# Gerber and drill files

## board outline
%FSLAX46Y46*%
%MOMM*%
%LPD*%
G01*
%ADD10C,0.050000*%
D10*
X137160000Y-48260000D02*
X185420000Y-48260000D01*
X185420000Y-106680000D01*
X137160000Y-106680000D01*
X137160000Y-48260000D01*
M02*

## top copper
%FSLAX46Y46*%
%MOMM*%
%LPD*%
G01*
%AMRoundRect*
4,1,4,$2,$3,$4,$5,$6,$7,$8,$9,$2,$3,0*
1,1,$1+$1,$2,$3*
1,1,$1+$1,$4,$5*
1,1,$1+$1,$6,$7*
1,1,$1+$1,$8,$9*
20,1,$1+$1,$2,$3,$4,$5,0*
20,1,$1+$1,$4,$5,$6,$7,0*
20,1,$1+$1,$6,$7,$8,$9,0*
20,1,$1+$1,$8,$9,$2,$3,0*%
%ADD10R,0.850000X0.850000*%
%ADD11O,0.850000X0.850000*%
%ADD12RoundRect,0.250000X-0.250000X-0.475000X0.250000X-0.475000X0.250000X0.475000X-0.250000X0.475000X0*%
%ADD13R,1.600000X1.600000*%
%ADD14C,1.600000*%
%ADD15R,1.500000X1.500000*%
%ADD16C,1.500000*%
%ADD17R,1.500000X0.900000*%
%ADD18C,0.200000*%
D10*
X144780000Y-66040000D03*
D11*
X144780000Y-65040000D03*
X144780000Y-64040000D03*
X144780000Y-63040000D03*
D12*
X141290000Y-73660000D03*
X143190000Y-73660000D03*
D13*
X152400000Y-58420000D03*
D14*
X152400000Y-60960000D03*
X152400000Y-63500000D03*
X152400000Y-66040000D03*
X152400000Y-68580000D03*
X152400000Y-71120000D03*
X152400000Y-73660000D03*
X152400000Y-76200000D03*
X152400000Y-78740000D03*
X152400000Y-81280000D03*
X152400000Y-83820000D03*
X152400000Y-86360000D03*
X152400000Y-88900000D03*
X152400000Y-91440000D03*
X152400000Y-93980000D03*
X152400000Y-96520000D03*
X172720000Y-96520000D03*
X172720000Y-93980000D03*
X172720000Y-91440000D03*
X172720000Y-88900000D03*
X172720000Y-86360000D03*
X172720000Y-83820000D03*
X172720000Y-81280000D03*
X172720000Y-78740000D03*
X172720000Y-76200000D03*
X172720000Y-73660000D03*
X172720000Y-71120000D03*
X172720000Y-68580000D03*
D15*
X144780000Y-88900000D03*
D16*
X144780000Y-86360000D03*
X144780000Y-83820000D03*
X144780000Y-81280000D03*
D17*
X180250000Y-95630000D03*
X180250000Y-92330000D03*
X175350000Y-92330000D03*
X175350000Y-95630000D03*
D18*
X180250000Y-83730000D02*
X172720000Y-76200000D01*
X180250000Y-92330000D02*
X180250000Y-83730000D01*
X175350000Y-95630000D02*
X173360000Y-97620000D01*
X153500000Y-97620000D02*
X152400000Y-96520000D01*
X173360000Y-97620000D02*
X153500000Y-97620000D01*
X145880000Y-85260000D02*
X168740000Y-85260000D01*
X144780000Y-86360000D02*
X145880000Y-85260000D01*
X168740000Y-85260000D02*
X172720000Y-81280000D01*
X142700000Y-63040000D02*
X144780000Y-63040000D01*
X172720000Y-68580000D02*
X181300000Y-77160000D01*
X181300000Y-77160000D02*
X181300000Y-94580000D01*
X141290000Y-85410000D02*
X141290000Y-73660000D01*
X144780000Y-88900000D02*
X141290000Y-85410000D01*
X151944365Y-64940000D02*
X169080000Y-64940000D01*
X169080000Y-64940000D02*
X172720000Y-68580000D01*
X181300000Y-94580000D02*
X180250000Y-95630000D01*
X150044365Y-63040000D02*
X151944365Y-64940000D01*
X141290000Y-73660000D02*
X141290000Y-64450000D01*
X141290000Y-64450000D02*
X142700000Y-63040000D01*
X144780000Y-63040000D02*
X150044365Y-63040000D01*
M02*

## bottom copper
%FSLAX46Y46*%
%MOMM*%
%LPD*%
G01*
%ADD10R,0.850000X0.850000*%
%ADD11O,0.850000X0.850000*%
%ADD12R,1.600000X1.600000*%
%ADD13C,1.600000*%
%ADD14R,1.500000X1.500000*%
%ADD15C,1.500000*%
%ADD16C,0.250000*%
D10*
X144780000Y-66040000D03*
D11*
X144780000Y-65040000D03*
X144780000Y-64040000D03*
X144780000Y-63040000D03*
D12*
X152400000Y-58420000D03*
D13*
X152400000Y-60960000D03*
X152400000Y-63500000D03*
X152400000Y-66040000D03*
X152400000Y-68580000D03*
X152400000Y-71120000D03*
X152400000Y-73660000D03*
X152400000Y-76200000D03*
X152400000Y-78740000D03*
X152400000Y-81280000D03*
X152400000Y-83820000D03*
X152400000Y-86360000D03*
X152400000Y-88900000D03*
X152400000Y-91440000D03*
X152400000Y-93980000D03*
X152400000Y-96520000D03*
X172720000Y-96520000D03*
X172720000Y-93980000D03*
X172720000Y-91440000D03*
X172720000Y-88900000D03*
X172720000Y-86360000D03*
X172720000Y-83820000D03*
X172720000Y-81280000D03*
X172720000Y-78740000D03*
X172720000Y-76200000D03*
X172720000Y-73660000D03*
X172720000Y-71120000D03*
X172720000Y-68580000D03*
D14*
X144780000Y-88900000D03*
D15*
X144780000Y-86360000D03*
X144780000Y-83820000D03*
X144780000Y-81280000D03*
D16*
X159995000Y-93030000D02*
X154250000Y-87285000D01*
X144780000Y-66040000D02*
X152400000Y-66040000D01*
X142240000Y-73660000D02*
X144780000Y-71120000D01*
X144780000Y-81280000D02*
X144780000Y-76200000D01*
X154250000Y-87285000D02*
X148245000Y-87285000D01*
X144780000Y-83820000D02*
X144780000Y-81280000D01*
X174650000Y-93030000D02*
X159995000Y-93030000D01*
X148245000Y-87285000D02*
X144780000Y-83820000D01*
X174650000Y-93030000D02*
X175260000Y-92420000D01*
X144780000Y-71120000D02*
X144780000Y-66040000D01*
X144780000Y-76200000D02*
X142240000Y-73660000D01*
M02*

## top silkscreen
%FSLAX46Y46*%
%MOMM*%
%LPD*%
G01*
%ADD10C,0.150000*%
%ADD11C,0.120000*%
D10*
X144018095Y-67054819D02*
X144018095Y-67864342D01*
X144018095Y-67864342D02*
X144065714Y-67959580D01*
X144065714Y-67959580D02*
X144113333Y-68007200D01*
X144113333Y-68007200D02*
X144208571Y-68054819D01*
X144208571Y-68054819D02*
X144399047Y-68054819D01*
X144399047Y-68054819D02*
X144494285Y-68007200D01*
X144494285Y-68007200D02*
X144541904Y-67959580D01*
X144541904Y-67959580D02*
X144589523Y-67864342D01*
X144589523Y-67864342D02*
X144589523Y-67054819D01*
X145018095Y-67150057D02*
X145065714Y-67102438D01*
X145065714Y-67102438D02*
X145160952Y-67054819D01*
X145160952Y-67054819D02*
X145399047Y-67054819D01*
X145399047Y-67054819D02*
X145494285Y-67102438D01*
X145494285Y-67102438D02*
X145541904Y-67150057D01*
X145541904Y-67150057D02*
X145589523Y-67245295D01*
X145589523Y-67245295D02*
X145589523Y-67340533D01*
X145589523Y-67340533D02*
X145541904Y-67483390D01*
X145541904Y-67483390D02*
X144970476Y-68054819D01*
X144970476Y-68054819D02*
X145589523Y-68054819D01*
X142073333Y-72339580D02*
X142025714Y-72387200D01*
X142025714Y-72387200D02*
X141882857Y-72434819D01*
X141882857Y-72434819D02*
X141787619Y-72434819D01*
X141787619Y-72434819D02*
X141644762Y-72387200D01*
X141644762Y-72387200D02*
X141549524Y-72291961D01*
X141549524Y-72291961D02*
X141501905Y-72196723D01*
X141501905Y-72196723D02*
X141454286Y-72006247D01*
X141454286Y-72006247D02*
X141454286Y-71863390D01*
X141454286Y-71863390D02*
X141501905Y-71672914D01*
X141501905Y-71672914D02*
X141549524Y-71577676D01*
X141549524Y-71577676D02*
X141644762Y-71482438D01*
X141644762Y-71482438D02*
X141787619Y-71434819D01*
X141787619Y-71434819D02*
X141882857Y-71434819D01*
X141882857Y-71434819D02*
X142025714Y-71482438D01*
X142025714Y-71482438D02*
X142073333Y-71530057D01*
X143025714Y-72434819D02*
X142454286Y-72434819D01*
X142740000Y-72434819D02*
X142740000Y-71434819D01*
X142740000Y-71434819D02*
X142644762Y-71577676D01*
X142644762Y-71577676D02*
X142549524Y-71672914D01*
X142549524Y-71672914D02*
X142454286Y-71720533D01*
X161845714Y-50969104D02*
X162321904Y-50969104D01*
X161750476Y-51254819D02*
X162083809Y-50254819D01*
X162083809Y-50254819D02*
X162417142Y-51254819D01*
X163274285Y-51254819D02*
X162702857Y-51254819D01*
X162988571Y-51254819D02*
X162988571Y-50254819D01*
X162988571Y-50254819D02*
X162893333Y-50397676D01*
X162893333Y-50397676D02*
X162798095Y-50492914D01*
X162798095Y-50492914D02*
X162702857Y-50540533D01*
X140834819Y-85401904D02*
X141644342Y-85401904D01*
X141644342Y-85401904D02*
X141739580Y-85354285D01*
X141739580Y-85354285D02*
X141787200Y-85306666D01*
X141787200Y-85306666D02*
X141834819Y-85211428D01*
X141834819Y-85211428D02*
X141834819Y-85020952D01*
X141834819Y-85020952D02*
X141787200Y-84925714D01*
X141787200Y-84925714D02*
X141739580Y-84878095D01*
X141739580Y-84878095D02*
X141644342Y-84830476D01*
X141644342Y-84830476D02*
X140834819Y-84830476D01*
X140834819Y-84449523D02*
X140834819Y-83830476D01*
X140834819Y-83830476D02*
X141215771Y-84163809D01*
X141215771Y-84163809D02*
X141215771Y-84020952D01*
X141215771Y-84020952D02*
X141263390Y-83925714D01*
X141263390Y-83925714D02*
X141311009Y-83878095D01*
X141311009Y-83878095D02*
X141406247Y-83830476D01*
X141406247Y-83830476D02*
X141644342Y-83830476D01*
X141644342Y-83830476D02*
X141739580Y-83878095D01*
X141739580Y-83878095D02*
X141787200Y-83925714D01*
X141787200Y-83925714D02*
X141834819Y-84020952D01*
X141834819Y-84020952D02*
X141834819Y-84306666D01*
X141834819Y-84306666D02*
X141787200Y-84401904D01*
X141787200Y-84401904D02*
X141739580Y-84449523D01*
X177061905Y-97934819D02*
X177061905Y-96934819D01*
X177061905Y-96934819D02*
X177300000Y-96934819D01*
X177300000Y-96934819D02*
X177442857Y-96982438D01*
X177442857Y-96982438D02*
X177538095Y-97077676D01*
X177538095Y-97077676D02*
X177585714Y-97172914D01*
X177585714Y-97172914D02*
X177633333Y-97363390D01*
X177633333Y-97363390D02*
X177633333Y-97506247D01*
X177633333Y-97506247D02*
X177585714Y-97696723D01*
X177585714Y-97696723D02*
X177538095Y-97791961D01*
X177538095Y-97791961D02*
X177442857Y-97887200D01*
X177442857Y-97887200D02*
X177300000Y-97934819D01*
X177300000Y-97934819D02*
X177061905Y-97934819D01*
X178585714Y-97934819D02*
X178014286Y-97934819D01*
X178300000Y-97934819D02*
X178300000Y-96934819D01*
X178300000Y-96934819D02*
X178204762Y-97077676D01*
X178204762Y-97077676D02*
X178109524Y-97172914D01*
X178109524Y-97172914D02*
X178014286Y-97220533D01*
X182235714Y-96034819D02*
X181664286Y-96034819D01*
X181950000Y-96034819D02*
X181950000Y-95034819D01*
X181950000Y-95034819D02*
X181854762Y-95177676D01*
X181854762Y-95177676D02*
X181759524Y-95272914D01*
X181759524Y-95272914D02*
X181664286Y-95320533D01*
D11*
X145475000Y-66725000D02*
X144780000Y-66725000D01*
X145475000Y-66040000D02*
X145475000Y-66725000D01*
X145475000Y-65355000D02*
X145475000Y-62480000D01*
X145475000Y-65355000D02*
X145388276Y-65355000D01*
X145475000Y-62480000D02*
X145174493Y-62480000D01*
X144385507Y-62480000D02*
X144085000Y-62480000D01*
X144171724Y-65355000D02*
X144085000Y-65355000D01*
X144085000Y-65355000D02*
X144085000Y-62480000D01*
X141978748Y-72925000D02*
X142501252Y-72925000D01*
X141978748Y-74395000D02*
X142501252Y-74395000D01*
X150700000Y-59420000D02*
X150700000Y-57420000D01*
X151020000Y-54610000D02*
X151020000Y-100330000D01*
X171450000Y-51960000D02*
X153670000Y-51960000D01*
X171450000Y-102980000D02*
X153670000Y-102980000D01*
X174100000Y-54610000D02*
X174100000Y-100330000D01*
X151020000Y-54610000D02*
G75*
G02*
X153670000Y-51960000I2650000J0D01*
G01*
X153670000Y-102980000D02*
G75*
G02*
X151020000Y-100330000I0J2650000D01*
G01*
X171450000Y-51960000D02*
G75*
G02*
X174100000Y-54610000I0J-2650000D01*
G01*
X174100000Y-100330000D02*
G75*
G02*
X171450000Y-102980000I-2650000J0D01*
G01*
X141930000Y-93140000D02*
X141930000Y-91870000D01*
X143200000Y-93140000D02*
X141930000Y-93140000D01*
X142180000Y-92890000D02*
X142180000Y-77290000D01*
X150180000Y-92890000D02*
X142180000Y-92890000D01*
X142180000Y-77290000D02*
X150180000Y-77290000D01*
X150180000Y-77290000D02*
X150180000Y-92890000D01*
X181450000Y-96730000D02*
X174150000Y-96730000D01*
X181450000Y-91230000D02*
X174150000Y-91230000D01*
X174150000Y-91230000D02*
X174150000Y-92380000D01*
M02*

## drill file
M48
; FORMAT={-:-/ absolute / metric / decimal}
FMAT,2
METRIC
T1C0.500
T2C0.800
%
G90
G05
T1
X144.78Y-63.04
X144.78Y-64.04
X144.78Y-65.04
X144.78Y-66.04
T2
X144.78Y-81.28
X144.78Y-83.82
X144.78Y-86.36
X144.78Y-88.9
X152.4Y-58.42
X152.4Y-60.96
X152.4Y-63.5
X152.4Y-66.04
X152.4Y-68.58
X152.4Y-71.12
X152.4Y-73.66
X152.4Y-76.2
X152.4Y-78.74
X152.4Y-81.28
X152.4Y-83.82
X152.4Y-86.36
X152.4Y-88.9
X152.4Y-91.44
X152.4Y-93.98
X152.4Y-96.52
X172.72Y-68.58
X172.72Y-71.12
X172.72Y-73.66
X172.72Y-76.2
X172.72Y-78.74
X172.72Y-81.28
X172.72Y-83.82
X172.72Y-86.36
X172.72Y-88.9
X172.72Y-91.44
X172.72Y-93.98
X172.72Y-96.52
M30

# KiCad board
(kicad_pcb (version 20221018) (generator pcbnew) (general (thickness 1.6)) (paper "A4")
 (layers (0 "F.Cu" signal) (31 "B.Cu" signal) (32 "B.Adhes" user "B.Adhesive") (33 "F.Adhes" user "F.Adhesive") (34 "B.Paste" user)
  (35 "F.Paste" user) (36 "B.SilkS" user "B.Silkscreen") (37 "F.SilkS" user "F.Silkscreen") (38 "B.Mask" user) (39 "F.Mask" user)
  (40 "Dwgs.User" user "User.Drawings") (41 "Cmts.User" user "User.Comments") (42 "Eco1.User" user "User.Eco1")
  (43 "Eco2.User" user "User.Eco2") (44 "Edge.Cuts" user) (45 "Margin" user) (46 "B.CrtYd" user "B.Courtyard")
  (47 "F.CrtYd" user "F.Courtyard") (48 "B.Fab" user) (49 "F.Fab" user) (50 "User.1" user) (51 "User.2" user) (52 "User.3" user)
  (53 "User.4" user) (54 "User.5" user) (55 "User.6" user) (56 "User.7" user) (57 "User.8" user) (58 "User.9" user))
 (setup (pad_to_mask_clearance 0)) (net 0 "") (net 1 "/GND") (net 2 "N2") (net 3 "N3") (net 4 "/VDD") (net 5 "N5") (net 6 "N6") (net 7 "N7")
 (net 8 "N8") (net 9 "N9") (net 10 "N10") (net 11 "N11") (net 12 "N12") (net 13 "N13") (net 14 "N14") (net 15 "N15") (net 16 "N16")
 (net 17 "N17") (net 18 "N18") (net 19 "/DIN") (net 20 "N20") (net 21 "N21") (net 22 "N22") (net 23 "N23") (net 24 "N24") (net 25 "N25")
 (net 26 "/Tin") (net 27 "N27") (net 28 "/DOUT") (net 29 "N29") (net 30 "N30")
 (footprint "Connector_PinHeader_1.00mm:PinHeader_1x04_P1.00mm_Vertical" (layer "F.Cu") (at 144.78 66.04 180)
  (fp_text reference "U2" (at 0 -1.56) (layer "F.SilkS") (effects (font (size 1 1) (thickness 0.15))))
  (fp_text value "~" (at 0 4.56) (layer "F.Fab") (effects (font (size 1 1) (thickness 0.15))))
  (fp_line (start -0.695 -0.685) (end 0 -0.685) (stroke (width 0.12) (type solid)) (layer "F.SilkS"))
  (fp_line (start -0.695 0) (end -0.695 -0.685) (stroke (width 0.12) (type solid)) (layer "F.SilkS"))
  (fp_line (start -0.695 0.685) (end -0.695 3.56) (stroke (width 0.12) (type solid)) (layer "F.SilkS"))
  (fp_line (start -0.695 0.685) (end -0.608276 0.685) (stroke (width 0.12) (type solid)) (layer "F.SilkS"))
  (fp_line (start -0.695 3.56) (end -0.394493 3.56) (stroke (width 0.12) (type solid)) (layer "F.SilkS"))
  (fp_line (start 0.394493 3.56) (end 0.695 3.56) (stroke (width 0.12) (type solid)) (layer "F.SilkS"))
  (fp_line (start 0.608276 0.685) (end 0.695 0.685) (stroke (width 0.12) (type solid)) (layer "F.SilkS"))
  (fp_line (start 0.695 0.685) (end 0.695 3.56) (stroke (width 0.12) (type solid)) (layer "F.SilkS"))
  (pad "1" thru_hole rect (at 0 0 180) (size 0.85 0.85) (drill 0.5) (layers "*.Cu" "*.Mask") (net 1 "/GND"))
  (pad "2" thru_hole oval (at 0 1 180) (size 0.85 0.85) (drill 0.5) (layers "*.Cu" "*.Mask") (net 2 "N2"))
  (pad "3" thru_hole oval (at 0 2 180) (size 0.85 0.85) (drill 0.5) (layers "*.Cu" "*.Mask") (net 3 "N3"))
  (pad "4" thru_hole oval (at 0 3 180) (size 0.85 0.85) (drill 0.5) (layers "*.Cu" "*.Mask") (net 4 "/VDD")))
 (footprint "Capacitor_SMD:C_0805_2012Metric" (layer "F.Cu") (at 142.24 73.66)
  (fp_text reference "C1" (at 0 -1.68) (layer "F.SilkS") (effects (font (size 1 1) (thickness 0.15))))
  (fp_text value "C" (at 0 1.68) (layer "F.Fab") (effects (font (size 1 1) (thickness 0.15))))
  (fp_line (start -0.261252 -0.735) (end 0.261252 -0.735) (stroke (width 0.12) (type solid)) (layer "F.SilkS"))
  (fp_line (start -0.261252 0.735) (end 0.261252 0.735) (stroke (width 0.12) (type solid)) (layer "F.SilkS"))
  (pad "1" smd roundrect (at -0.95 0) (size 1 1.45) (layers "F.Cu" "F.Paste" "F.Mask") (roundrect_rratio 0.25) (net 4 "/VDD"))
  (pad "2" smd roundrect (at 0.95 0) (size 1 1.45) (layers "F.Cu" "F.Paste" "F.Mask") (roundrect_rratio 0.25) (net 1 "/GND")))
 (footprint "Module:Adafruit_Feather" (layer "F.Cu") (at 152.4 58.42)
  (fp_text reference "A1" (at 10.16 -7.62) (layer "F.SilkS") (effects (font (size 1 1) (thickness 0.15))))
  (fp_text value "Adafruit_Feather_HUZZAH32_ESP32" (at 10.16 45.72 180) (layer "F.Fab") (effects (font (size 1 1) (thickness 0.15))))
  (fp_line (start -1.7 1) (end -1.7 -1) (stroke (width 0.12) (type solid)) (layer "F.SilkS"))
  (fp_line (start -1.38 -3.81) (end -1.38 41.91) (stroke (width 0.12) (type solid)) (layer "F.SilkS"))
  (fp_line (start 19.05 -6.46) (end 1.27 -6.46) (stroke (width 0.12) (type solid)) (layer "F.SilkS"))
  (fp_line (start 19.05 44.56) (end 1.27 44.56) (stroke (width 0.12) (type solid)) (layer "F.SilkS"))
  (fp_line (start 21.7 -3.81) (end 21.7 41.91) (stroke (width 0.12) (type solid)) (layer "F.SilkS"))
  (fp_arc (start -1.38 -3.81) (mid -0.603833 -5.683833) (end 1.27 -6.46) (stroke (width 0.12) (type solid)) (layer "F.SilkS"))
  (fp_arc (start 1.27 44.56) (mid -0.603833 43.783833) (end -1.38 41.91) (stroke (width 0.12) (type solid)) (layer "F.SilkS"))
  (fp_arc (start 19.05 -6.46) (mid 20.923833 -5.683833) (end 21.7 -3.81) (stroke (width 0.12) (type solid)) (layer "F.SilkS"))
  (fp_arc (start 21.7 41.91) (mid 20.923833 43.783833) (end 19.05 44.56) (stroke (width 0.12) (type solid)) (layer "F.SilkS"))
  (pad "1" thru_hole rect (at 0 0 180) (size 1.6 1.6) (drill 0.8) (layers "*.Cu" "*.Mask") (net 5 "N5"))
  (pad "2" thru_hole circle (at 0 2.54 180) (size 1.6 1.6) (drill 0.8) (layers "*.Cu" "*.Mask") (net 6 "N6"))
  (pad "3" thru_hole circle (at 0 5.08 180) (size 1.6 1.6) (drill 0.8) (layers "*.Cu" "*.Mask") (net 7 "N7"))
  (pad "4" thru_hole circle (at 0 7.62 180) (size 1.6 1.6) (drill 0.8) (layers "*.Cu" "*.Mask") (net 1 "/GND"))
  (pad "5" thru_hole circle (at 0 10.16 180) (size 1.6 1.6) (drill 0.8) (layers "*.Cu" "*.Mask") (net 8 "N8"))
  (pad "6" thru_hole circle (at 0 12.7 180) (size 1.6 1.6) (drill 0.8) (layers "*.Cu" "*.Mask") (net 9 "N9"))
  (pad "7" thru_hole circle (at 0 15.24 180) (size 1.6 1.6) (drill 0.8) (layers "*.Cu" "*.Mask") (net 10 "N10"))
  (pad "8" thru_hole circle (at 0 17.78 180) (size 1.6 1.6) (drill 0.8) (layers "*.Cu" "*.Mask") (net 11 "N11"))
  (pad "9" thru_hole circle (at 0 20.32 180) (size 1.6 1.6) (drill 0.8) (layers "*.Cu" "*.Mask") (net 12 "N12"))
  (pad "10" thru_hole circle (at 0 22.86 180) (size 1.6 1.6) (drill 0.8) (layers "*.Cu" "*.Mask") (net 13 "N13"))
  (pad "11" thru_hole circle (at 0 25.4 180) (size 1.6 1.6) (drill 0.8) (layers "*.Cu" "*.Mask") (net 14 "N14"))
  (pad "12" thru_hole circle (at 0 27.94 180) (size 1.6 1.6) (drill 0.8) (layers "*.Cu" "*.Mask") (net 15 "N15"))
  (pad "13" thru_hole circle (at 0 30.48 180) (size 1.6 1.6) (drill 0.8) (layers "*.Cu" "*.Mask") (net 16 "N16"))
  (pad "14" thru_hole circle (at 0 33.02 180) (size 1.6 1.6) (drill 0.8) (layers "*.Cu" "*.Mask") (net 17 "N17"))
  (pad "15" thru_hole circle (at 0 35.56 180) (size 1.6 1.6) (drill 0.8) (layers "*.Cu" "*.Mask") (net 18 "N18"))
  (pad "16" thru_hole circle (at 0 38.1 180) (size 1.6 1.6) (drill 0.8) (layers "*.Cu" "*.Mask") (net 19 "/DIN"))
  (pad "17" thru_hole circle (at 20.32 38.1 180) (size 1.6 1.6) (drill 0.8) (layers "*.Cu" "*.Mask") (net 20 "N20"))
  (pad "18" thru_hole circle (at 20.32 35.56 180) (size 1.6 1.6) (drill 0.8) (layers "*.Cu" "*.Mask") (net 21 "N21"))
  (pad "19" thru_hole circle (at 20.32 33.02 180) (size 1.6 1.6) (drill 0.8) (layers "*.Cu" "*.Mask") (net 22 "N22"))
  (pad "20" thru_hole circle (at 20.32 30.48 180) (size 1.6 1.6) (drill 0.8) (layers "*.Cu" "*.Mask") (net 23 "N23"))
  (pad "21" thru_hole circle (at 20.32 27.94 180) (size 1.6 1.6) (drill 0.8) (layers "*.Cu" "*.Mask") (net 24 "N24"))
  (pad "22" thru_hole circle (at 20.32 25.4 180) (size 1.6 1.6) (drill 0.8) (layers "*.Cu" "*.Mask") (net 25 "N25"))
  (pad "23" thru_hole circle (at 20.32 22.86 180) (size 1.6 1.6) (drill 0.8) (layers "*.Cu" "*.Mask") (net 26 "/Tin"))
  (pad "24" thru_hole circle (at 20.32 20.32 180) (size 1.6 1.6) (drill 0.8) (layers "*.Cu" "*.Mask") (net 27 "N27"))
  (pad "25" thru_hole circle (at 20.32 17.78 180) (size 1.6 1.6) (drill 0.8) (layers "*.Cu" "*.Mask") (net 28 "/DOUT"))
  (pad "26" thru_hole circle (at 20.32 15.24 180) (size 1.6 1.6) (drill 0.8) (layers "*.Cu" "*.Mask") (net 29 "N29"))
  (pad "27" thru_hole circle (at 20.32 12.7 180) (size 1.6 1.6) (drill 0.8) (layers "*.Cu" "*.Mask") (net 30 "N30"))
  (pad "28" thru_hole circle (at 20.32 10.16 180) (size 1.6 1.6) (drill 0.8) (layers "*.Cu" "*.Mask") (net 4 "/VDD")))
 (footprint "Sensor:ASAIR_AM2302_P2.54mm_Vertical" (layer "F.Cu") (at 144.78 88.9 90)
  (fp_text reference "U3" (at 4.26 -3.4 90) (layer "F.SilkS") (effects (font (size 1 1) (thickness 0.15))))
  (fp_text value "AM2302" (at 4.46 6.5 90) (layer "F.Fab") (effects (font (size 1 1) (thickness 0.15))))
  (fp_line (start -4.24 -2.85) (end -2.97 -2.85) (stroke (width 0.12) (type solid)) (layer "F.SilkS"))
  (fp_line (start -4.24 -1.58) (end -4.24 -2.85) (stroke (width 0.12) (type solid)) (layer "F.SilkS"))
  (fp_line (start -3.99 -2.6) (end 11.61 -2.6) (stroke (width 0.12) (type solid)) (layer "F.SilkS"))
  (fp_line (start -3.99 5.4) (end -3.99 -2.6) (stroke (width 0.12) (type solid)) (layer "F.SilkS"))
  (fp_line (start 11.61 -2.6) (end 11.61 5.4) (stroke (width 0.12) (type solid)) (layer "F.SilkS"))
  (fp_line (start 11.61 5.4) (end -3.99 5.4) (stroke (width 0.12) (type solid)) (layer "F.SilkS"))
  (pad "1" thru_hole rect (at 0 0 180) (size 1.5 1.5) (drill 0.8) (layers "*.Cu" "*.Mask") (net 4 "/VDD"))
  (pad "2" thru_hole circle (at 2.54 0 180) (size 1.5 1.5) (drill 0.8) (layers "*.Cu" "*.Mask") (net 26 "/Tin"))
  (pad "3" thru_hole circle (at 5.08 0 180) (size 1.5 1.5) (drill 0.8) (layers "*.Cu" "*.Mask") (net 1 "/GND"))
  (pad "4" thru_hole circle (at 7.62 0 180) (size 1.5 1.5) (drill 0.8) (layers "*.Cu" "*.Mask") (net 1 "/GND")))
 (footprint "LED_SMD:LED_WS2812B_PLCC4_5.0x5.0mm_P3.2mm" (layer "F.Cu") (at 177.8 93.98 180)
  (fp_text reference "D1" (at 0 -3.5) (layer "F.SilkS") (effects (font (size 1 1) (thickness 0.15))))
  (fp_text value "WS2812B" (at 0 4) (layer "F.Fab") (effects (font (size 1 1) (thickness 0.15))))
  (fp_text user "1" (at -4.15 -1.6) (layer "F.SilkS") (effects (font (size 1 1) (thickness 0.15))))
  (fp_line (start -3.65 -2.75) (end 3.65 -2.75) (stroke (width 0.12) (type solid)) (layer "F.SilkS"))
  (fp_line (start -3.65 2.75) (end 3.65 2.75) (stroke (width 0.12) (type solid)) (layer "F.SilkS"))
  (fp_line (start 3.65 2.75) (end 3.65 1.6) (stroke (width 0.12) (type solid)) (layer "F.SilkS"))
  (pad "1" smd rect (at -2.45 -1.65 180) (size 1.5 0.9) (layers "F.Cu" "F.Paste" "F.Mask") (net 4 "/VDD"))
  (pad "2" smd rect (at -2.45 1.65 180) (size 1.5 0.9) (layers "F.Cu" "F.Paste" "F.Mask") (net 28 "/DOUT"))
  (pad "3" smd rect (at 2.45 1.65 180) (size 1.5 0.9) (layers "F.Cu" "F.Paste" "F.Mask") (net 1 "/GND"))
  (pad "4" smd rect (at 2.45 -1.65 180) (size 1.5 0.9) (layers "F.Cu" "F.Paste" "F.Mask") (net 19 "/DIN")))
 (gr_rect (start 137.16 48.26) (end 185.42 106.68) (stroke (width 0.05) (type default)) (fill none) (layer "Edge.Cuts"))
 (segment (start 159.995 93.03) (end 154.25 87.285) (width 0.25) (layer "B.Cu") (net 1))
 (segment (start 144.78 66.04) (end 152.4 66.04) (width 0.25) (layer "B.Cu") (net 1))
 (segment (start 142.24 73.66) (end 144.78 71.12) (width 0.25) (layer "B.Cu") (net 1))
 (segment (start 144.78 81.28) (end 144.78 76.2) (width 0.25) (layer "B.Cu") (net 1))
 (segment (start 154.25 87.285) (end 148.245 87.285) (width 0.25) (layer "B.Cu") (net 1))
 (segment (start 144.78 83.82) (end 144.78 81.28) (width 0.25) (layer "B.Cu") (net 1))
 (segment (start 174.65 93.03) (end 159.995 93.03) (width 0.25) (layer "B.Cu") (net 1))
 (segment (start 148.245 87.285) (end 144.78 83.82) (width 0.25) (layer "B.Cu") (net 1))
 (segment (start 174.65 93.03) (end 175.26 92.42) (width 0.25) (layer "B.Cu") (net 1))
 (segment (start 144.78 71.12) (end 144.78 66.04) (width 0.25) (layer "B.Cu") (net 1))
 (segment (start 144.78 76.2) (end 142.24 73.66) (width 0.25) (layer "B.Cu") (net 1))
 (segment (start 180.25 83.73) (end 172.72 76.2) (width 0.2) (layer "F.Cu") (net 28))
 (segment (start 180.25 92.33) (end 180.25 83.73) (width 0.2) (layer "F.Cu") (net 28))
 (segment (start 175.35 95.63) (end 173.36 97.62) (width 0.2) (layer "F.Cu") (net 19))
 (segment (start 153.5 97.62) (end 152.4 96.52) (width 0.2) (layer "F.Cu") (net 19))
 (segment (start 173.36 97.62) (end 153.5 97.62) (width 0.2) (layer "F.Cu") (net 19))
 (segment (start 145.88 85.26) (end 168.74 85.26) (width 0.2) (layer "F.Cu") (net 26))
 (segment (start 144.78 86.36) (end 145.88 85.26) (width 0.2) (layer "F.Cu") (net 26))
 (segment (start 168.74 85.26) (end 172.72 81.28) (width 0.2) (layer "F.Cu") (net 26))
 (segment (start 142.7 63.04) (end 144.78 63.04) (width 0.2) (layer "F.Cu") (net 4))
 (segment (start 172.72 68.58) (end 181.3 77.16) (width 0.2) (layer "F.Cu") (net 4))
 (segment (start 181.3 77.16) (end 181.3 94.58) (width 0.2) (layer "F.Cu") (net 4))
 (segment (start 141.29 85.41) (end 141.29 73.66) (width 0.2) (layer "F.Cu") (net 4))
 (segment (start 144.78 88.9) (end 141.29 85.41) (width 0.2) (layer "F.Cu") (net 4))
 (segment (start 151.944365 64.94) (end 169.08 64.94) (width 0.2) (layer "F.Cu") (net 4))
 (segment (start 169.08 64.94) (end 172.72 68.58) (width 0.2) (layer "F.Cu") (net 4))
 (segment (start 181.3 94.58) (end 180.25 95.63) (width 0.2) (layer "F.Cu") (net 4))
 (segment (start 150.044365 63.04) (end 151.944365 64.94) (width 0.2) (layer "F.Cu") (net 4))
 (segment (start 141.29 73.66) (end 141.29 64.45) (width 0.2) (layer "F.Cu") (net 4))
 (segment (start 141.29 64.45) (end 142.7 63.04) (width 0.2) (layer "F.Cu") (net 4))
 (segment (start 144.78 63.04) (end 150.044365 63.04) (width 0.2) (layer "F.Cu") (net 4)))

